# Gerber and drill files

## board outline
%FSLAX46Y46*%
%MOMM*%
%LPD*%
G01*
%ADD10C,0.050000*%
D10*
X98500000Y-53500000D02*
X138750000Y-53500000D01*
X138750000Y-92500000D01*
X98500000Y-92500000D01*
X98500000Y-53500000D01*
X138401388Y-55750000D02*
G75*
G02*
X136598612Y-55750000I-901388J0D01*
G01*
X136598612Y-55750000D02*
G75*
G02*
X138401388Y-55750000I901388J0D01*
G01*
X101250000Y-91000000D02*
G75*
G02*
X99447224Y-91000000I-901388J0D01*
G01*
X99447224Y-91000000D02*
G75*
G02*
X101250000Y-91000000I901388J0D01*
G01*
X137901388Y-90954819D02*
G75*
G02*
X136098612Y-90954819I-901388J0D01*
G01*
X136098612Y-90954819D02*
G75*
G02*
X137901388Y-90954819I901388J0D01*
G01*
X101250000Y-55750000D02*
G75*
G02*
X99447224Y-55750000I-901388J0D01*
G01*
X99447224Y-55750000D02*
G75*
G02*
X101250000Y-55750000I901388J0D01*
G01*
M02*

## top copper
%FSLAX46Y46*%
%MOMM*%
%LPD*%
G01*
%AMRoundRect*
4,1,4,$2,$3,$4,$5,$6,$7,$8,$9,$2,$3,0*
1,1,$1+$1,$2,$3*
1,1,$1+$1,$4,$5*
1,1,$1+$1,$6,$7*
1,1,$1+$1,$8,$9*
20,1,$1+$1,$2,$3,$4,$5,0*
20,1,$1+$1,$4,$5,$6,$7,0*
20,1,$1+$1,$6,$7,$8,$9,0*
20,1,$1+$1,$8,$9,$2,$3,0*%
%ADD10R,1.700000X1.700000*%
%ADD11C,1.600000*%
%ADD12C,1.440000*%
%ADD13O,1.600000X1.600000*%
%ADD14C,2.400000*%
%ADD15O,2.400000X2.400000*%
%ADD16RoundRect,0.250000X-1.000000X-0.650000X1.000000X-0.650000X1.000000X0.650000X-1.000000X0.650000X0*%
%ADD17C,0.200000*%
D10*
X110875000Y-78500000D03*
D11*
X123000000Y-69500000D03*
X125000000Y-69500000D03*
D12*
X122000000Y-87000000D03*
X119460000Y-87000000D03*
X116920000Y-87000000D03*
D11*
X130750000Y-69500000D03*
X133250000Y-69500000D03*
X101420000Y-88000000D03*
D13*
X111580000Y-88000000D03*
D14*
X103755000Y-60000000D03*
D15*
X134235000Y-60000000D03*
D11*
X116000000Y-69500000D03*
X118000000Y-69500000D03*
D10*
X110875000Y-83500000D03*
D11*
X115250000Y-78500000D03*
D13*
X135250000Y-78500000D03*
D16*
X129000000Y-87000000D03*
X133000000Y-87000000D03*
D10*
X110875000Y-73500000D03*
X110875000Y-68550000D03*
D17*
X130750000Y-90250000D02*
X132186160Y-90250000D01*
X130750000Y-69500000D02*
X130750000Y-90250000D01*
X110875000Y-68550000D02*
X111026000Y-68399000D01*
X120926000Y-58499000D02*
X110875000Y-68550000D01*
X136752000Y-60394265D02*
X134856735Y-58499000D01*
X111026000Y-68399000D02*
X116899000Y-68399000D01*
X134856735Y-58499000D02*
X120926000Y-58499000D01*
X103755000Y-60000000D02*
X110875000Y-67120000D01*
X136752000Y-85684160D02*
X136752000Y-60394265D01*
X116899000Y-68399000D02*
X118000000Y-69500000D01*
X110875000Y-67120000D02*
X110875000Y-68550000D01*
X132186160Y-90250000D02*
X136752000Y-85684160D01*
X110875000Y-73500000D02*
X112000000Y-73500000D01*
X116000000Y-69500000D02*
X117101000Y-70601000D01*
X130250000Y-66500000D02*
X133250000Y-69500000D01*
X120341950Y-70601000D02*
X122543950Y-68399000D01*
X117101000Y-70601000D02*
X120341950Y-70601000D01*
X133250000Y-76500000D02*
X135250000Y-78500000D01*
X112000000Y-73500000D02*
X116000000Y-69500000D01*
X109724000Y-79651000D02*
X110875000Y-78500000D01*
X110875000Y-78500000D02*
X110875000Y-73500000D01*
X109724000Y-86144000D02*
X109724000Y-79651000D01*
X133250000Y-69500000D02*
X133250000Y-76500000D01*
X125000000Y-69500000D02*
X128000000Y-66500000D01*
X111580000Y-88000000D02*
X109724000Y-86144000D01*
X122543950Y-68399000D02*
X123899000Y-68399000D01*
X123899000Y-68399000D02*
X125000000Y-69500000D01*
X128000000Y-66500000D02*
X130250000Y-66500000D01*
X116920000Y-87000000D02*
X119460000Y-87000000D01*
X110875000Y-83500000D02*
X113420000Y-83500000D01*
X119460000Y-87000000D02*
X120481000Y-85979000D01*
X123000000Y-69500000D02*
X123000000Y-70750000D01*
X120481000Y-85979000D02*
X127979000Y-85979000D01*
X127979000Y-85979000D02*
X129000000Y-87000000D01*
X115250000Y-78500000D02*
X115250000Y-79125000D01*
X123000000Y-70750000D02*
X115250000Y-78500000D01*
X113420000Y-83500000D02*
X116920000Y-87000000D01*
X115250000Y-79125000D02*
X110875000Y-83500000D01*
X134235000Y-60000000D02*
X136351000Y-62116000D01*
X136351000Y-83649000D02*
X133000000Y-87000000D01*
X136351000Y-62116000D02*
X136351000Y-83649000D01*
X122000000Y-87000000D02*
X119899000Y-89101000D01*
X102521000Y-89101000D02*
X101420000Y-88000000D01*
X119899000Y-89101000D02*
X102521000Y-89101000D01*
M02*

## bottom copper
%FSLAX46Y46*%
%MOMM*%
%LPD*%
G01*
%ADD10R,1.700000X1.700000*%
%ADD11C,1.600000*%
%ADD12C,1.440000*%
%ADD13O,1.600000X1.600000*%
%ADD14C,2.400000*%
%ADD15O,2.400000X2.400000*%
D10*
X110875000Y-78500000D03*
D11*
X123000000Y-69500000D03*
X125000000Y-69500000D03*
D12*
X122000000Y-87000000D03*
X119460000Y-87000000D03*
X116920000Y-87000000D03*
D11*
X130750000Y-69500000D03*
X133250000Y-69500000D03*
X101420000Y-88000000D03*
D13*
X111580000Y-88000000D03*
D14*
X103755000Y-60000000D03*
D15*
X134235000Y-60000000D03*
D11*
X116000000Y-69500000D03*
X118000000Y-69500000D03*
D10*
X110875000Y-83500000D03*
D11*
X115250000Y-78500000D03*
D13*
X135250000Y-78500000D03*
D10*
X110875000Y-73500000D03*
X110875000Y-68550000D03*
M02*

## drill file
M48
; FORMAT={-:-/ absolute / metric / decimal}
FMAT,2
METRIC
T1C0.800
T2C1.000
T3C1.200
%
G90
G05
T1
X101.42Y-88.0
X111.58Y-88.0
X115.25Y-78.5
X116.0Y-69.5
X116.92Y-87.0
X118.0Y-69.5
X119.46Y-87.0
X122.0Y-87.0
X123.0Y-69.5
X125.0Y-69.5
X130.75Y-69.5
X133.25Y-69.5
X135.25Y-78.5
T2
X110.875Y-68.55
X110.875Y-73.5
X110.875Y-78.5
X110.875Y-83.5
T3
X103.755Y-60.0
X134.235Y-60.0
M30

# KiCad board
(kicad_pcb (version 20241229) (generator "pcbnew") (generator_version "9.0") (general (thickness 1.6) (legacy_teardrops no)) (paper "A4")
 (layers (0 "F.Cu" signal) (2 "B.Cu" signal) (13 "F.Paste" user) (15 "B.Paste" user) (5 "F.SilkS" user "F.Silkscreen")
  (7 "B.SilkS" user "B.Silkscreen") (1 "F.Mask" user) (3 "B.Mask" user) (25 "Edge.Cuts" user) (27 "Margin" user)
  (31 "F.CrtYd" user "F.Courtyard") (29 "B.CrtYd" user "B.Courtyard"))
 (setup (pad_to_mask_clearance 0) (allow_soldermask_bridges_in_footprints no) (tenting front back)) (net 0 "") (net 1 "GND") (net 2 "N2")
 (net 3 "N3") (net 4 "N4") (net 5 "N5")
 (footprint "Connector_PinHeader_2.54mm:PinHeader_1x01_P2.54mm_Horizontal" (layer "F.Cu") (at 110.875 78.5 180)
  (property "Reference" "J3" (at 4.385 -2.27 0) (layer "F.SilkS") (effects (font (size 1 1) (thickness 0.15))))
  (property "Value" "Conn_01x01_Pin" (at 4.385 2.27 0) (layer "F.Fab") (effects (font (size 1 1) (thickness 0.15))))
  (pad "1" thru_hole rect (at 0 0 180) (size 1.7 1.7) (drill 1) (layers "*.Cu" "*.Mask") (remove_unused_layers no) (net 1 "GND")))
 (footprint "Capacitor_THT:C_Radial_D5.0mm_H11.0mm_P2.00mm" (layer "F.Cu") (at 123 69.5)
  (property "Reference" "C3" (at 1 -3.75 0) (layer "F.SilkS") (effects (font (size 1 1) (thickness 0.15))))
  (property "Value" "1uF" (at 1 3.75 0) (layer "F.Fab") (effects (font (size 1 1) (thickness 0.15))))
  (pad "1" thru_hole circle (at 0 0) (size 1.6 1.6) (drill 0.8) (layers "*.Cu" "*.Mask") (remove_unused_layers no) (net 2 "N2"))
  (pad "2" thru_hole circle (at 2 0) (size 1.6 1.6) (drill 0.8) (layers "*.Cu" "*.Mask") (remove_unused_layers no) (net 1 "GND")))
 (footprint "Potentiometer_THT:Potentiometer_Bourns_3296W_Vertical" (layer "F.Cu") (at 122 87)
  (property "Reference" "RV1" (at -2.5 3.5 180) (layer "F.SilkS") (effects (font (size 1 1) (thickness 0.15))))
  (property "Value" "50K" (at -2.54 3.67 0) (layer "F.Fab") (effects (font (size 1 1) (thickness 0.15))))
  (pad "1" thru_hole circle (at 0 0) (size 1.44 1.44) (drill 0.8) (layers "*.Cu" "*.Mask") (remove_unused_layers no) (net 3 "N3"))
  (pad "2" thru_hole circle (at -2.54 0) (size 1.44 1.44) (drill 0.8) (layers "*.Cu" "*.Mask") (remove_unused_layers no) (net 2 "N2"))
  (pad "3" thru_hole circle (at -5.08 0) (size 1.44 1.44) (drill 0.8) (layers "*.Cu" "*.Mask") (remove_unused_layers no) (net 2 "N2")))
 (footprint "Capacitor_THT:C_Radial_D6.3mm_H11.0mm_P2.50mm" (layer "F.Cu") (at 130.75 69.5)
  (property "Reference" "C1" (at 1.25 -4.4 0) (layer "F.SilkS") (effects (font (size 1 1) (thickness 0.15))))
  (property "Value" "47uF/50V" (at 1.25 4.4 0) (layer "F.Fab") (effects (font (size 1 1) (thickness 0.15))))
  (pad "1" thru_hole circle (at 0 0) (size 1.6 1.6) (drill 0.8) (layers "*.Cu" "*.Mask") (remove_unused_layers no) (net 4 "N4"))
  (pad "2" thru_hole circle (at 2.5 0) (size 1.6 1.6) (drill 0.8) (layers "*.Cu" "*.Mask") (remove_unused_layers no) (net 1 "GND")))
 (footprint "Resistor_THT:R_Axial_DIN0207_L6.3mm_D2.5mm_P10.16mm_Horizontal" (layer "F.Cu") (at 101.42 88)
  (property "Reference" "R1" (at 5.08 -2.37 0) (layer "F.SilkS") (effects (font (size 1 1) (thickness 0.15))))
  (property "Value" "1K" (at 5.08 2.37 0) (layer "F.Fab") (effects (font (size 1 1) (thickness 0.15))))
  (pad "1" thru_hole circle (at 0 0) (size 1.6 1.6) (drill 0.8) (layers "*.Cu" "*.Mask") (remove_unused_layers no) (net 3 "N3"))
  (pad "2" thru_hole oval (at 10.16 0) (size 1.6 1.6) (drill 0.8) (layers "*.Cu" "*.Mask") (remove_unused_layers no) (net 1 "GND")))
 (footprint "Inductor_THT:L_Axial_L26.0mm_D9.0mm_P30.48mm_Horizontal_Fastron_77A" (layer "F.Cu") (at 103.755 60)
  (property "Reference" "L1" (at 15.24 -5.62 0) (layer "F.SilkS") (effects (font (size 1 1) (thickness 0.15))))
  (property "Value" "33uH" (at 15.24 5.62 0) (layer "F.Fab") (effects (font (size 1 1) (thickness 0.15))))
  (pad "1" thru_hole circle (at 0 0) (size 2.4 2.4) (drill 1.2) (layers "*.Cu" "*.Mask") (remove_unused_layers no) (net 4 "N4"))
  (pad "2" thru_hole oval (at 30.48 0) (size 2.4 2.4) (drill 1.2) (layers "*.Cu" "*.Mask") (remove_unused_layers no) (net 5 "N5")))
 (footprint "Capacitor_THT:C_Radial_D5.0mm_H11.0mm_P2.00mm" (layer "F.Cu") (at 116 69.5)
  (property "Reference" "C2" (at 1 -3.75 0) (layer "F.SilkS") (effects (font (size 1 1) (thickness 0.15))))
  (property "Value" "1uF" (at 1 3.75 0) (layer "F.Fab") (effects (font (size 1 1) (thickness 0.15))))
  (pad "1" thru_hole circle (at 0 0) (size 1.6 1.6) (drill 0.8) (layers "*.Cu" "*.Mask") (remove_unused_layers no) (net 1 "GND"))
  (pad "2" thru_hole circle (at 2 0) (size 1.6 1.6) (drill 0.8) (layers "*.Cu" "*.Mask") (remove_unused_layers no) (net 4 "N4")))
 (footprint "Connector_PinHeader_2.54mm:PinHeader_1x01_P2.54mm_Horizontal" (layer "F.Cu") (at 110.875 83.5 180)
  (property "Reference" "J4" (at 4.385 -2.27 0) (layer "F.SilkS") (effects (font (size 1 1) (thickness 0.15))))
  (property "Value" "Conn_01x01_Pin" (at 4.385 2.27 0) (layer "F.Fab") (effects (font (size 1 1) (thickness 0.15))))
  (pad "1" thru_hole rect (at 0 0 180) (size 1.7 1.7) (drill 1) (layers "*.Cu" "*.Mask") (remove_unused_layers no) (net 2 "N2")))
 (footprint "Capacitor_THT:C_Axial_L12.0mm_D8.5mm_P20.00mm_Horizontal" (layer "F.Cu") (at 115.25 78.5)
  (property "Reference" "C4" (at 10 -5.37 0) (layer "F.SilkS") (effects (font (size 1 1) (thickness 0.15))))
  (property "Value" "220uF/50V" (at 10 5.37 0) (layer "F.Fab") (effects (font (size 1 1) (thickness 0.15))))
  (pad "1" thru_hole circle (at 0 0) (size 1.6 1.6) (drill 0.8) (layers "*.Cu" "*.Mask") (remove_unused_layers no) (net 2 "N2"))
  (pad "2" thru_hole oval (at 20 0) (size 1.6 1.6) (drill 0.8) (layers "*.Cu" "*.Mask") (remove_unused_layers no) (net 1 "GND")))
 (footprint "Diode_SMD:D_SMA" (layer "F.Cu") (at 131 87)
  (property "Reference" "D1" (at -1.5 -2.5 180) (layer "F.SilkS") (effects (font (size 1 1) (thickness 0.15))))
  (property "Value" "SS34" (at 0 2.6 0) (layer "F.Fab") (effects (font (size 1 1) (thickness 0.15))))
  (pad "1" smd roundrect (at -2 0) (size 2.5 1.8) (layers "F.Cu" "F.Mask" "F.Paste") (roundrect_rratio 0.1388888889) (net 2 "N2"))
  (pad "2" smd roundrect (at 2 0) (size 2.5 1.8) (layers "F.Cu" "F.Mask" "F.Paste") (roundrect_rratio 0.1388888889) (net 5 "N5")))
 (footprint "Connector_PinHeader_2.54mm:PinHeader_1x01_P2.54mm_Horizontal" (layer "F.Cu") (at 110.875 73.5 180)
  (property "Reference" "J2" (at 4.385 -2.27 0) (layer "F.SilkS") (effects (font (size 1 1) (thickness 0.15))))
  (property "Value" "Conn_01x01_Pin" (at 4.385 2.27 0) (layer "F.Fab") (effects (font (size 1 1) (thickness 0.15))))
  (pad "1" thru_hole rect (at 0 0 180) (size 1.7 1.7) (drill 1) (layers "*.Cu" "*.Mask") (remove_unused_layers no) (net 1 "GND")))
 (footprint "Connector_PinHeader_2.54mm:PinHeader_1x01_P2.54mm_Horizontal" (layer "F.Cu") (at 110.875 68.55 180)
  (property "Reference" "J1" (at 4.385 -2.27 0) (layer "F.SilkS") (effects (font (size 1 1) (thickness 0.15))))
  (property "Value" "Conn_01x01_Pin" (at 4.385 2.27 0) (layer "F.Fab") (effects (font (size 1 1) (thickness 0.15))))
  (pad "1" thru_hole rect (at 0 0 180) (size 1.7 1.7) (drill 1) (layers "*.Cu" "*.Mask") (remove_unused_layers no) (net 4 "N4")))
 (gr_rect (start 98.5 53.5) (end 138.75 92.5) (stroke (width 0.05) (type default)) (fill no) (layer "Edge.Cuts"))
 (gr_circle (center 137.5 55.75) (end 138.25 56.25) (stroke (width 0.05) (type default)) (fill no) (layer "Edge.Cuts"))
 (gr_circle (center 100.348612 91) (end 101.098612 91.5) (stroke (width 0.05) (type default)) (fill no) (layer "Edge.Cuts"))
 (gr_circle (center 137 90.954819) (end 137.75 91.454819) (stroke (width 0.05) (type default)) (fill no) (layer "Edge.Cuts"))
 (gr_circle (center 100.348612 55.75) (end 101.098612 56.25) (stroke (width 0.05) (type default)) (fill no) (layer "Edge.Cuts"))
 (segment (start 130.75 90.25) (end 132.18616 90.25) (width 0.2) (layer "F.Cu") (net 4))
 (segment (start 130.75 69.5) (end 130.75 90.25) (width 0.2) (layer "F.Cu") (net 4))
 (segment (start 110.875 68.55) (end 111.026 68.399) (width 0.2) (layer "F.Cu") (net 4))
 (segment (start 120.926 58.499) (end 110.875 68.55) (width 0.2) (layer "F.Cu") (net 4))
 (segment (start 136.752 60.394265) (end 134.856735 58.499) (width 0.2) (layer "F.Cu") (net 4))
 (segment (start 111.026 68.399) (end 116.899 68.399) (width 0.2) (layer "F.Cu") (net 4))
 (segment (start 134.856735 58.499) (end 120.926 58.499) (width 0.2) (layer "F.Cu") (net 4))
 (segment (start 103.755 60) (end 110.875 67.12) (width 0.2) (layer "F.Cu") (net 4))
 (segment (start 136.752 85.68416) (end 136.752 60.394265) (width 0.2) (layer "F.Cu") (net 4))
 (segment (start 116.899 68.399) (end 118 69.5) (width 0.2) (layer "F.Cu") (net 4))
 (segment (start 110.875 67.12) (end 110.875 68.55) (width 0.2) (layer "F.Cu") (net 4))
 (segment (start 132.18616 90.25) (end 136.752 85.68416) (width 0.2) (layer "F.Cu") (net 4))
 (segment (start 110.875 73.5) (end 112 73.5) (width 0.2) (layer "F.Cu") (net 1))
 (segment (start 116 69.5) (end 117.101 70.601) (width 0.2) (layer "F.Cu") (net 1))
 (segment (start 130.25 66.5) (end 133.25 69.5) (width 0.2) (layer "F.Cu") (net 1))
 (segment (start 120.34195 70.601) (end 122.54395 68.399) (width 0.2) (layer "F.Cu") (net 1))
 (segment (start 117.101 70.601) (end 120.34195 70.601) (width 0.2) (layer "F.Cu") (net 1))
 (segment (start 133.25 76.5) (end 135.25 78.5) (width 0.2) (layer "F.Cu") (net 1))
 (segment (start 112 73.5) (end 116 69.5) (width 0.2) (layer "F.Cu") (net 1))
 (segment (start 109.724 79.651) (end 110.875 78.5) (width 0.2) (layer "F.Cu") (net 1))
 (segment (start 110.875 78.5) (end 110.875 73.5) (width 0.2) (layer "F.Cu") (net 1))
 (segment (start 109.724 86.144) (end 109.724 79.651) (width 0.2) (layer "F.Cu") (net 1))
 (segment (start 133.25 69.5) (end 133.25 76.5) (width 0.2) (layer "F.Cu") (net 1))
 (segment (start 125 69.5) (end 128 66.5) (width 0.2) (layer "F.Cu") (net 1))
 (segment (start 111.58 88) (end 109.724 86.144) (width 0.2) (layer "F.Cu") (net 1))
 (segment (start 122.54395 68.399) (end 123.899 68.399) (width 0.2) (layer "F.Cu") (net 1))
 (segment (start 123.899 68.399) (end 125 69.5) (width 0.2) (layer "F.Cu") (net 1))
 (segment (start 128 66.5) (end 130.25 66.5) (width 0.2) (layer "F.Cu") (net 1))
 (segment (start 116.92 87) (end 119.46 87) (width 0.2) (layer "F.Cu") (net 2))
 (segment (start 110.875 83.5) (end 113.42 83.5) (width 0.2) (layer "F.Cu") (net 2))
 (segment (start 119.46 87) (end 120.481 85.979) (width 0.2) (layer "F.Cu") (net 2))
 (segment (start 123 69.5) (end 123 70.75) (width 0.2) (layer "F.Cu") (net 2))
 (segment (start 120.481 85.979) (end 127.979 85.979) (width 0.2) (layer "F.Cu") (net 2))
 (segment (start 127.979 85.979) (end 129 87) (width 0.2) (layer "F.Cu") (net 2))
 (segment (start 115.25 78.5) (end 115.25 79.125) (width 0.2) (layer "F.Cu") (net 2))
 (segment (start 123 70.75) (end 115.25 78.5) (width 0.2) (layer "F.Cu") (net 2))
 (segment (start 113.42 83.5) (end 116.92 87) (width 0.2) (layer "F.Cu") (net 2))
 (segment (start 115.25 79.125) (end 110.875 83.5) (width 0.2) (layer "F.Cu") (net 2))
 (segment (start 134.235 60) (end 136.351 62.116) (width 0.2) (layer "F.Cu") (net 5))
 (segment (start 136.351 83.649) (end 133 87) (width 0.2) (layer "F.Cu") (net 5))
 (segment (start 136.351 62.116) (end 136.351 83.649) (width 0.2) (layer "F.Cu") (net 5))
 (segment (start 122 87) (end 119.899 89.101) (width 0.2) (layer "F.Cu") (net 3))
 (segment (start 102.521 89.101) (end 101.42 88) (width 0.2) (layer "F.Cu") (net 3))
 (segment (start 119.899 89.101) (end 102.521 89.101) (width 0.2) (layer "F.Cu") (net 3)))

